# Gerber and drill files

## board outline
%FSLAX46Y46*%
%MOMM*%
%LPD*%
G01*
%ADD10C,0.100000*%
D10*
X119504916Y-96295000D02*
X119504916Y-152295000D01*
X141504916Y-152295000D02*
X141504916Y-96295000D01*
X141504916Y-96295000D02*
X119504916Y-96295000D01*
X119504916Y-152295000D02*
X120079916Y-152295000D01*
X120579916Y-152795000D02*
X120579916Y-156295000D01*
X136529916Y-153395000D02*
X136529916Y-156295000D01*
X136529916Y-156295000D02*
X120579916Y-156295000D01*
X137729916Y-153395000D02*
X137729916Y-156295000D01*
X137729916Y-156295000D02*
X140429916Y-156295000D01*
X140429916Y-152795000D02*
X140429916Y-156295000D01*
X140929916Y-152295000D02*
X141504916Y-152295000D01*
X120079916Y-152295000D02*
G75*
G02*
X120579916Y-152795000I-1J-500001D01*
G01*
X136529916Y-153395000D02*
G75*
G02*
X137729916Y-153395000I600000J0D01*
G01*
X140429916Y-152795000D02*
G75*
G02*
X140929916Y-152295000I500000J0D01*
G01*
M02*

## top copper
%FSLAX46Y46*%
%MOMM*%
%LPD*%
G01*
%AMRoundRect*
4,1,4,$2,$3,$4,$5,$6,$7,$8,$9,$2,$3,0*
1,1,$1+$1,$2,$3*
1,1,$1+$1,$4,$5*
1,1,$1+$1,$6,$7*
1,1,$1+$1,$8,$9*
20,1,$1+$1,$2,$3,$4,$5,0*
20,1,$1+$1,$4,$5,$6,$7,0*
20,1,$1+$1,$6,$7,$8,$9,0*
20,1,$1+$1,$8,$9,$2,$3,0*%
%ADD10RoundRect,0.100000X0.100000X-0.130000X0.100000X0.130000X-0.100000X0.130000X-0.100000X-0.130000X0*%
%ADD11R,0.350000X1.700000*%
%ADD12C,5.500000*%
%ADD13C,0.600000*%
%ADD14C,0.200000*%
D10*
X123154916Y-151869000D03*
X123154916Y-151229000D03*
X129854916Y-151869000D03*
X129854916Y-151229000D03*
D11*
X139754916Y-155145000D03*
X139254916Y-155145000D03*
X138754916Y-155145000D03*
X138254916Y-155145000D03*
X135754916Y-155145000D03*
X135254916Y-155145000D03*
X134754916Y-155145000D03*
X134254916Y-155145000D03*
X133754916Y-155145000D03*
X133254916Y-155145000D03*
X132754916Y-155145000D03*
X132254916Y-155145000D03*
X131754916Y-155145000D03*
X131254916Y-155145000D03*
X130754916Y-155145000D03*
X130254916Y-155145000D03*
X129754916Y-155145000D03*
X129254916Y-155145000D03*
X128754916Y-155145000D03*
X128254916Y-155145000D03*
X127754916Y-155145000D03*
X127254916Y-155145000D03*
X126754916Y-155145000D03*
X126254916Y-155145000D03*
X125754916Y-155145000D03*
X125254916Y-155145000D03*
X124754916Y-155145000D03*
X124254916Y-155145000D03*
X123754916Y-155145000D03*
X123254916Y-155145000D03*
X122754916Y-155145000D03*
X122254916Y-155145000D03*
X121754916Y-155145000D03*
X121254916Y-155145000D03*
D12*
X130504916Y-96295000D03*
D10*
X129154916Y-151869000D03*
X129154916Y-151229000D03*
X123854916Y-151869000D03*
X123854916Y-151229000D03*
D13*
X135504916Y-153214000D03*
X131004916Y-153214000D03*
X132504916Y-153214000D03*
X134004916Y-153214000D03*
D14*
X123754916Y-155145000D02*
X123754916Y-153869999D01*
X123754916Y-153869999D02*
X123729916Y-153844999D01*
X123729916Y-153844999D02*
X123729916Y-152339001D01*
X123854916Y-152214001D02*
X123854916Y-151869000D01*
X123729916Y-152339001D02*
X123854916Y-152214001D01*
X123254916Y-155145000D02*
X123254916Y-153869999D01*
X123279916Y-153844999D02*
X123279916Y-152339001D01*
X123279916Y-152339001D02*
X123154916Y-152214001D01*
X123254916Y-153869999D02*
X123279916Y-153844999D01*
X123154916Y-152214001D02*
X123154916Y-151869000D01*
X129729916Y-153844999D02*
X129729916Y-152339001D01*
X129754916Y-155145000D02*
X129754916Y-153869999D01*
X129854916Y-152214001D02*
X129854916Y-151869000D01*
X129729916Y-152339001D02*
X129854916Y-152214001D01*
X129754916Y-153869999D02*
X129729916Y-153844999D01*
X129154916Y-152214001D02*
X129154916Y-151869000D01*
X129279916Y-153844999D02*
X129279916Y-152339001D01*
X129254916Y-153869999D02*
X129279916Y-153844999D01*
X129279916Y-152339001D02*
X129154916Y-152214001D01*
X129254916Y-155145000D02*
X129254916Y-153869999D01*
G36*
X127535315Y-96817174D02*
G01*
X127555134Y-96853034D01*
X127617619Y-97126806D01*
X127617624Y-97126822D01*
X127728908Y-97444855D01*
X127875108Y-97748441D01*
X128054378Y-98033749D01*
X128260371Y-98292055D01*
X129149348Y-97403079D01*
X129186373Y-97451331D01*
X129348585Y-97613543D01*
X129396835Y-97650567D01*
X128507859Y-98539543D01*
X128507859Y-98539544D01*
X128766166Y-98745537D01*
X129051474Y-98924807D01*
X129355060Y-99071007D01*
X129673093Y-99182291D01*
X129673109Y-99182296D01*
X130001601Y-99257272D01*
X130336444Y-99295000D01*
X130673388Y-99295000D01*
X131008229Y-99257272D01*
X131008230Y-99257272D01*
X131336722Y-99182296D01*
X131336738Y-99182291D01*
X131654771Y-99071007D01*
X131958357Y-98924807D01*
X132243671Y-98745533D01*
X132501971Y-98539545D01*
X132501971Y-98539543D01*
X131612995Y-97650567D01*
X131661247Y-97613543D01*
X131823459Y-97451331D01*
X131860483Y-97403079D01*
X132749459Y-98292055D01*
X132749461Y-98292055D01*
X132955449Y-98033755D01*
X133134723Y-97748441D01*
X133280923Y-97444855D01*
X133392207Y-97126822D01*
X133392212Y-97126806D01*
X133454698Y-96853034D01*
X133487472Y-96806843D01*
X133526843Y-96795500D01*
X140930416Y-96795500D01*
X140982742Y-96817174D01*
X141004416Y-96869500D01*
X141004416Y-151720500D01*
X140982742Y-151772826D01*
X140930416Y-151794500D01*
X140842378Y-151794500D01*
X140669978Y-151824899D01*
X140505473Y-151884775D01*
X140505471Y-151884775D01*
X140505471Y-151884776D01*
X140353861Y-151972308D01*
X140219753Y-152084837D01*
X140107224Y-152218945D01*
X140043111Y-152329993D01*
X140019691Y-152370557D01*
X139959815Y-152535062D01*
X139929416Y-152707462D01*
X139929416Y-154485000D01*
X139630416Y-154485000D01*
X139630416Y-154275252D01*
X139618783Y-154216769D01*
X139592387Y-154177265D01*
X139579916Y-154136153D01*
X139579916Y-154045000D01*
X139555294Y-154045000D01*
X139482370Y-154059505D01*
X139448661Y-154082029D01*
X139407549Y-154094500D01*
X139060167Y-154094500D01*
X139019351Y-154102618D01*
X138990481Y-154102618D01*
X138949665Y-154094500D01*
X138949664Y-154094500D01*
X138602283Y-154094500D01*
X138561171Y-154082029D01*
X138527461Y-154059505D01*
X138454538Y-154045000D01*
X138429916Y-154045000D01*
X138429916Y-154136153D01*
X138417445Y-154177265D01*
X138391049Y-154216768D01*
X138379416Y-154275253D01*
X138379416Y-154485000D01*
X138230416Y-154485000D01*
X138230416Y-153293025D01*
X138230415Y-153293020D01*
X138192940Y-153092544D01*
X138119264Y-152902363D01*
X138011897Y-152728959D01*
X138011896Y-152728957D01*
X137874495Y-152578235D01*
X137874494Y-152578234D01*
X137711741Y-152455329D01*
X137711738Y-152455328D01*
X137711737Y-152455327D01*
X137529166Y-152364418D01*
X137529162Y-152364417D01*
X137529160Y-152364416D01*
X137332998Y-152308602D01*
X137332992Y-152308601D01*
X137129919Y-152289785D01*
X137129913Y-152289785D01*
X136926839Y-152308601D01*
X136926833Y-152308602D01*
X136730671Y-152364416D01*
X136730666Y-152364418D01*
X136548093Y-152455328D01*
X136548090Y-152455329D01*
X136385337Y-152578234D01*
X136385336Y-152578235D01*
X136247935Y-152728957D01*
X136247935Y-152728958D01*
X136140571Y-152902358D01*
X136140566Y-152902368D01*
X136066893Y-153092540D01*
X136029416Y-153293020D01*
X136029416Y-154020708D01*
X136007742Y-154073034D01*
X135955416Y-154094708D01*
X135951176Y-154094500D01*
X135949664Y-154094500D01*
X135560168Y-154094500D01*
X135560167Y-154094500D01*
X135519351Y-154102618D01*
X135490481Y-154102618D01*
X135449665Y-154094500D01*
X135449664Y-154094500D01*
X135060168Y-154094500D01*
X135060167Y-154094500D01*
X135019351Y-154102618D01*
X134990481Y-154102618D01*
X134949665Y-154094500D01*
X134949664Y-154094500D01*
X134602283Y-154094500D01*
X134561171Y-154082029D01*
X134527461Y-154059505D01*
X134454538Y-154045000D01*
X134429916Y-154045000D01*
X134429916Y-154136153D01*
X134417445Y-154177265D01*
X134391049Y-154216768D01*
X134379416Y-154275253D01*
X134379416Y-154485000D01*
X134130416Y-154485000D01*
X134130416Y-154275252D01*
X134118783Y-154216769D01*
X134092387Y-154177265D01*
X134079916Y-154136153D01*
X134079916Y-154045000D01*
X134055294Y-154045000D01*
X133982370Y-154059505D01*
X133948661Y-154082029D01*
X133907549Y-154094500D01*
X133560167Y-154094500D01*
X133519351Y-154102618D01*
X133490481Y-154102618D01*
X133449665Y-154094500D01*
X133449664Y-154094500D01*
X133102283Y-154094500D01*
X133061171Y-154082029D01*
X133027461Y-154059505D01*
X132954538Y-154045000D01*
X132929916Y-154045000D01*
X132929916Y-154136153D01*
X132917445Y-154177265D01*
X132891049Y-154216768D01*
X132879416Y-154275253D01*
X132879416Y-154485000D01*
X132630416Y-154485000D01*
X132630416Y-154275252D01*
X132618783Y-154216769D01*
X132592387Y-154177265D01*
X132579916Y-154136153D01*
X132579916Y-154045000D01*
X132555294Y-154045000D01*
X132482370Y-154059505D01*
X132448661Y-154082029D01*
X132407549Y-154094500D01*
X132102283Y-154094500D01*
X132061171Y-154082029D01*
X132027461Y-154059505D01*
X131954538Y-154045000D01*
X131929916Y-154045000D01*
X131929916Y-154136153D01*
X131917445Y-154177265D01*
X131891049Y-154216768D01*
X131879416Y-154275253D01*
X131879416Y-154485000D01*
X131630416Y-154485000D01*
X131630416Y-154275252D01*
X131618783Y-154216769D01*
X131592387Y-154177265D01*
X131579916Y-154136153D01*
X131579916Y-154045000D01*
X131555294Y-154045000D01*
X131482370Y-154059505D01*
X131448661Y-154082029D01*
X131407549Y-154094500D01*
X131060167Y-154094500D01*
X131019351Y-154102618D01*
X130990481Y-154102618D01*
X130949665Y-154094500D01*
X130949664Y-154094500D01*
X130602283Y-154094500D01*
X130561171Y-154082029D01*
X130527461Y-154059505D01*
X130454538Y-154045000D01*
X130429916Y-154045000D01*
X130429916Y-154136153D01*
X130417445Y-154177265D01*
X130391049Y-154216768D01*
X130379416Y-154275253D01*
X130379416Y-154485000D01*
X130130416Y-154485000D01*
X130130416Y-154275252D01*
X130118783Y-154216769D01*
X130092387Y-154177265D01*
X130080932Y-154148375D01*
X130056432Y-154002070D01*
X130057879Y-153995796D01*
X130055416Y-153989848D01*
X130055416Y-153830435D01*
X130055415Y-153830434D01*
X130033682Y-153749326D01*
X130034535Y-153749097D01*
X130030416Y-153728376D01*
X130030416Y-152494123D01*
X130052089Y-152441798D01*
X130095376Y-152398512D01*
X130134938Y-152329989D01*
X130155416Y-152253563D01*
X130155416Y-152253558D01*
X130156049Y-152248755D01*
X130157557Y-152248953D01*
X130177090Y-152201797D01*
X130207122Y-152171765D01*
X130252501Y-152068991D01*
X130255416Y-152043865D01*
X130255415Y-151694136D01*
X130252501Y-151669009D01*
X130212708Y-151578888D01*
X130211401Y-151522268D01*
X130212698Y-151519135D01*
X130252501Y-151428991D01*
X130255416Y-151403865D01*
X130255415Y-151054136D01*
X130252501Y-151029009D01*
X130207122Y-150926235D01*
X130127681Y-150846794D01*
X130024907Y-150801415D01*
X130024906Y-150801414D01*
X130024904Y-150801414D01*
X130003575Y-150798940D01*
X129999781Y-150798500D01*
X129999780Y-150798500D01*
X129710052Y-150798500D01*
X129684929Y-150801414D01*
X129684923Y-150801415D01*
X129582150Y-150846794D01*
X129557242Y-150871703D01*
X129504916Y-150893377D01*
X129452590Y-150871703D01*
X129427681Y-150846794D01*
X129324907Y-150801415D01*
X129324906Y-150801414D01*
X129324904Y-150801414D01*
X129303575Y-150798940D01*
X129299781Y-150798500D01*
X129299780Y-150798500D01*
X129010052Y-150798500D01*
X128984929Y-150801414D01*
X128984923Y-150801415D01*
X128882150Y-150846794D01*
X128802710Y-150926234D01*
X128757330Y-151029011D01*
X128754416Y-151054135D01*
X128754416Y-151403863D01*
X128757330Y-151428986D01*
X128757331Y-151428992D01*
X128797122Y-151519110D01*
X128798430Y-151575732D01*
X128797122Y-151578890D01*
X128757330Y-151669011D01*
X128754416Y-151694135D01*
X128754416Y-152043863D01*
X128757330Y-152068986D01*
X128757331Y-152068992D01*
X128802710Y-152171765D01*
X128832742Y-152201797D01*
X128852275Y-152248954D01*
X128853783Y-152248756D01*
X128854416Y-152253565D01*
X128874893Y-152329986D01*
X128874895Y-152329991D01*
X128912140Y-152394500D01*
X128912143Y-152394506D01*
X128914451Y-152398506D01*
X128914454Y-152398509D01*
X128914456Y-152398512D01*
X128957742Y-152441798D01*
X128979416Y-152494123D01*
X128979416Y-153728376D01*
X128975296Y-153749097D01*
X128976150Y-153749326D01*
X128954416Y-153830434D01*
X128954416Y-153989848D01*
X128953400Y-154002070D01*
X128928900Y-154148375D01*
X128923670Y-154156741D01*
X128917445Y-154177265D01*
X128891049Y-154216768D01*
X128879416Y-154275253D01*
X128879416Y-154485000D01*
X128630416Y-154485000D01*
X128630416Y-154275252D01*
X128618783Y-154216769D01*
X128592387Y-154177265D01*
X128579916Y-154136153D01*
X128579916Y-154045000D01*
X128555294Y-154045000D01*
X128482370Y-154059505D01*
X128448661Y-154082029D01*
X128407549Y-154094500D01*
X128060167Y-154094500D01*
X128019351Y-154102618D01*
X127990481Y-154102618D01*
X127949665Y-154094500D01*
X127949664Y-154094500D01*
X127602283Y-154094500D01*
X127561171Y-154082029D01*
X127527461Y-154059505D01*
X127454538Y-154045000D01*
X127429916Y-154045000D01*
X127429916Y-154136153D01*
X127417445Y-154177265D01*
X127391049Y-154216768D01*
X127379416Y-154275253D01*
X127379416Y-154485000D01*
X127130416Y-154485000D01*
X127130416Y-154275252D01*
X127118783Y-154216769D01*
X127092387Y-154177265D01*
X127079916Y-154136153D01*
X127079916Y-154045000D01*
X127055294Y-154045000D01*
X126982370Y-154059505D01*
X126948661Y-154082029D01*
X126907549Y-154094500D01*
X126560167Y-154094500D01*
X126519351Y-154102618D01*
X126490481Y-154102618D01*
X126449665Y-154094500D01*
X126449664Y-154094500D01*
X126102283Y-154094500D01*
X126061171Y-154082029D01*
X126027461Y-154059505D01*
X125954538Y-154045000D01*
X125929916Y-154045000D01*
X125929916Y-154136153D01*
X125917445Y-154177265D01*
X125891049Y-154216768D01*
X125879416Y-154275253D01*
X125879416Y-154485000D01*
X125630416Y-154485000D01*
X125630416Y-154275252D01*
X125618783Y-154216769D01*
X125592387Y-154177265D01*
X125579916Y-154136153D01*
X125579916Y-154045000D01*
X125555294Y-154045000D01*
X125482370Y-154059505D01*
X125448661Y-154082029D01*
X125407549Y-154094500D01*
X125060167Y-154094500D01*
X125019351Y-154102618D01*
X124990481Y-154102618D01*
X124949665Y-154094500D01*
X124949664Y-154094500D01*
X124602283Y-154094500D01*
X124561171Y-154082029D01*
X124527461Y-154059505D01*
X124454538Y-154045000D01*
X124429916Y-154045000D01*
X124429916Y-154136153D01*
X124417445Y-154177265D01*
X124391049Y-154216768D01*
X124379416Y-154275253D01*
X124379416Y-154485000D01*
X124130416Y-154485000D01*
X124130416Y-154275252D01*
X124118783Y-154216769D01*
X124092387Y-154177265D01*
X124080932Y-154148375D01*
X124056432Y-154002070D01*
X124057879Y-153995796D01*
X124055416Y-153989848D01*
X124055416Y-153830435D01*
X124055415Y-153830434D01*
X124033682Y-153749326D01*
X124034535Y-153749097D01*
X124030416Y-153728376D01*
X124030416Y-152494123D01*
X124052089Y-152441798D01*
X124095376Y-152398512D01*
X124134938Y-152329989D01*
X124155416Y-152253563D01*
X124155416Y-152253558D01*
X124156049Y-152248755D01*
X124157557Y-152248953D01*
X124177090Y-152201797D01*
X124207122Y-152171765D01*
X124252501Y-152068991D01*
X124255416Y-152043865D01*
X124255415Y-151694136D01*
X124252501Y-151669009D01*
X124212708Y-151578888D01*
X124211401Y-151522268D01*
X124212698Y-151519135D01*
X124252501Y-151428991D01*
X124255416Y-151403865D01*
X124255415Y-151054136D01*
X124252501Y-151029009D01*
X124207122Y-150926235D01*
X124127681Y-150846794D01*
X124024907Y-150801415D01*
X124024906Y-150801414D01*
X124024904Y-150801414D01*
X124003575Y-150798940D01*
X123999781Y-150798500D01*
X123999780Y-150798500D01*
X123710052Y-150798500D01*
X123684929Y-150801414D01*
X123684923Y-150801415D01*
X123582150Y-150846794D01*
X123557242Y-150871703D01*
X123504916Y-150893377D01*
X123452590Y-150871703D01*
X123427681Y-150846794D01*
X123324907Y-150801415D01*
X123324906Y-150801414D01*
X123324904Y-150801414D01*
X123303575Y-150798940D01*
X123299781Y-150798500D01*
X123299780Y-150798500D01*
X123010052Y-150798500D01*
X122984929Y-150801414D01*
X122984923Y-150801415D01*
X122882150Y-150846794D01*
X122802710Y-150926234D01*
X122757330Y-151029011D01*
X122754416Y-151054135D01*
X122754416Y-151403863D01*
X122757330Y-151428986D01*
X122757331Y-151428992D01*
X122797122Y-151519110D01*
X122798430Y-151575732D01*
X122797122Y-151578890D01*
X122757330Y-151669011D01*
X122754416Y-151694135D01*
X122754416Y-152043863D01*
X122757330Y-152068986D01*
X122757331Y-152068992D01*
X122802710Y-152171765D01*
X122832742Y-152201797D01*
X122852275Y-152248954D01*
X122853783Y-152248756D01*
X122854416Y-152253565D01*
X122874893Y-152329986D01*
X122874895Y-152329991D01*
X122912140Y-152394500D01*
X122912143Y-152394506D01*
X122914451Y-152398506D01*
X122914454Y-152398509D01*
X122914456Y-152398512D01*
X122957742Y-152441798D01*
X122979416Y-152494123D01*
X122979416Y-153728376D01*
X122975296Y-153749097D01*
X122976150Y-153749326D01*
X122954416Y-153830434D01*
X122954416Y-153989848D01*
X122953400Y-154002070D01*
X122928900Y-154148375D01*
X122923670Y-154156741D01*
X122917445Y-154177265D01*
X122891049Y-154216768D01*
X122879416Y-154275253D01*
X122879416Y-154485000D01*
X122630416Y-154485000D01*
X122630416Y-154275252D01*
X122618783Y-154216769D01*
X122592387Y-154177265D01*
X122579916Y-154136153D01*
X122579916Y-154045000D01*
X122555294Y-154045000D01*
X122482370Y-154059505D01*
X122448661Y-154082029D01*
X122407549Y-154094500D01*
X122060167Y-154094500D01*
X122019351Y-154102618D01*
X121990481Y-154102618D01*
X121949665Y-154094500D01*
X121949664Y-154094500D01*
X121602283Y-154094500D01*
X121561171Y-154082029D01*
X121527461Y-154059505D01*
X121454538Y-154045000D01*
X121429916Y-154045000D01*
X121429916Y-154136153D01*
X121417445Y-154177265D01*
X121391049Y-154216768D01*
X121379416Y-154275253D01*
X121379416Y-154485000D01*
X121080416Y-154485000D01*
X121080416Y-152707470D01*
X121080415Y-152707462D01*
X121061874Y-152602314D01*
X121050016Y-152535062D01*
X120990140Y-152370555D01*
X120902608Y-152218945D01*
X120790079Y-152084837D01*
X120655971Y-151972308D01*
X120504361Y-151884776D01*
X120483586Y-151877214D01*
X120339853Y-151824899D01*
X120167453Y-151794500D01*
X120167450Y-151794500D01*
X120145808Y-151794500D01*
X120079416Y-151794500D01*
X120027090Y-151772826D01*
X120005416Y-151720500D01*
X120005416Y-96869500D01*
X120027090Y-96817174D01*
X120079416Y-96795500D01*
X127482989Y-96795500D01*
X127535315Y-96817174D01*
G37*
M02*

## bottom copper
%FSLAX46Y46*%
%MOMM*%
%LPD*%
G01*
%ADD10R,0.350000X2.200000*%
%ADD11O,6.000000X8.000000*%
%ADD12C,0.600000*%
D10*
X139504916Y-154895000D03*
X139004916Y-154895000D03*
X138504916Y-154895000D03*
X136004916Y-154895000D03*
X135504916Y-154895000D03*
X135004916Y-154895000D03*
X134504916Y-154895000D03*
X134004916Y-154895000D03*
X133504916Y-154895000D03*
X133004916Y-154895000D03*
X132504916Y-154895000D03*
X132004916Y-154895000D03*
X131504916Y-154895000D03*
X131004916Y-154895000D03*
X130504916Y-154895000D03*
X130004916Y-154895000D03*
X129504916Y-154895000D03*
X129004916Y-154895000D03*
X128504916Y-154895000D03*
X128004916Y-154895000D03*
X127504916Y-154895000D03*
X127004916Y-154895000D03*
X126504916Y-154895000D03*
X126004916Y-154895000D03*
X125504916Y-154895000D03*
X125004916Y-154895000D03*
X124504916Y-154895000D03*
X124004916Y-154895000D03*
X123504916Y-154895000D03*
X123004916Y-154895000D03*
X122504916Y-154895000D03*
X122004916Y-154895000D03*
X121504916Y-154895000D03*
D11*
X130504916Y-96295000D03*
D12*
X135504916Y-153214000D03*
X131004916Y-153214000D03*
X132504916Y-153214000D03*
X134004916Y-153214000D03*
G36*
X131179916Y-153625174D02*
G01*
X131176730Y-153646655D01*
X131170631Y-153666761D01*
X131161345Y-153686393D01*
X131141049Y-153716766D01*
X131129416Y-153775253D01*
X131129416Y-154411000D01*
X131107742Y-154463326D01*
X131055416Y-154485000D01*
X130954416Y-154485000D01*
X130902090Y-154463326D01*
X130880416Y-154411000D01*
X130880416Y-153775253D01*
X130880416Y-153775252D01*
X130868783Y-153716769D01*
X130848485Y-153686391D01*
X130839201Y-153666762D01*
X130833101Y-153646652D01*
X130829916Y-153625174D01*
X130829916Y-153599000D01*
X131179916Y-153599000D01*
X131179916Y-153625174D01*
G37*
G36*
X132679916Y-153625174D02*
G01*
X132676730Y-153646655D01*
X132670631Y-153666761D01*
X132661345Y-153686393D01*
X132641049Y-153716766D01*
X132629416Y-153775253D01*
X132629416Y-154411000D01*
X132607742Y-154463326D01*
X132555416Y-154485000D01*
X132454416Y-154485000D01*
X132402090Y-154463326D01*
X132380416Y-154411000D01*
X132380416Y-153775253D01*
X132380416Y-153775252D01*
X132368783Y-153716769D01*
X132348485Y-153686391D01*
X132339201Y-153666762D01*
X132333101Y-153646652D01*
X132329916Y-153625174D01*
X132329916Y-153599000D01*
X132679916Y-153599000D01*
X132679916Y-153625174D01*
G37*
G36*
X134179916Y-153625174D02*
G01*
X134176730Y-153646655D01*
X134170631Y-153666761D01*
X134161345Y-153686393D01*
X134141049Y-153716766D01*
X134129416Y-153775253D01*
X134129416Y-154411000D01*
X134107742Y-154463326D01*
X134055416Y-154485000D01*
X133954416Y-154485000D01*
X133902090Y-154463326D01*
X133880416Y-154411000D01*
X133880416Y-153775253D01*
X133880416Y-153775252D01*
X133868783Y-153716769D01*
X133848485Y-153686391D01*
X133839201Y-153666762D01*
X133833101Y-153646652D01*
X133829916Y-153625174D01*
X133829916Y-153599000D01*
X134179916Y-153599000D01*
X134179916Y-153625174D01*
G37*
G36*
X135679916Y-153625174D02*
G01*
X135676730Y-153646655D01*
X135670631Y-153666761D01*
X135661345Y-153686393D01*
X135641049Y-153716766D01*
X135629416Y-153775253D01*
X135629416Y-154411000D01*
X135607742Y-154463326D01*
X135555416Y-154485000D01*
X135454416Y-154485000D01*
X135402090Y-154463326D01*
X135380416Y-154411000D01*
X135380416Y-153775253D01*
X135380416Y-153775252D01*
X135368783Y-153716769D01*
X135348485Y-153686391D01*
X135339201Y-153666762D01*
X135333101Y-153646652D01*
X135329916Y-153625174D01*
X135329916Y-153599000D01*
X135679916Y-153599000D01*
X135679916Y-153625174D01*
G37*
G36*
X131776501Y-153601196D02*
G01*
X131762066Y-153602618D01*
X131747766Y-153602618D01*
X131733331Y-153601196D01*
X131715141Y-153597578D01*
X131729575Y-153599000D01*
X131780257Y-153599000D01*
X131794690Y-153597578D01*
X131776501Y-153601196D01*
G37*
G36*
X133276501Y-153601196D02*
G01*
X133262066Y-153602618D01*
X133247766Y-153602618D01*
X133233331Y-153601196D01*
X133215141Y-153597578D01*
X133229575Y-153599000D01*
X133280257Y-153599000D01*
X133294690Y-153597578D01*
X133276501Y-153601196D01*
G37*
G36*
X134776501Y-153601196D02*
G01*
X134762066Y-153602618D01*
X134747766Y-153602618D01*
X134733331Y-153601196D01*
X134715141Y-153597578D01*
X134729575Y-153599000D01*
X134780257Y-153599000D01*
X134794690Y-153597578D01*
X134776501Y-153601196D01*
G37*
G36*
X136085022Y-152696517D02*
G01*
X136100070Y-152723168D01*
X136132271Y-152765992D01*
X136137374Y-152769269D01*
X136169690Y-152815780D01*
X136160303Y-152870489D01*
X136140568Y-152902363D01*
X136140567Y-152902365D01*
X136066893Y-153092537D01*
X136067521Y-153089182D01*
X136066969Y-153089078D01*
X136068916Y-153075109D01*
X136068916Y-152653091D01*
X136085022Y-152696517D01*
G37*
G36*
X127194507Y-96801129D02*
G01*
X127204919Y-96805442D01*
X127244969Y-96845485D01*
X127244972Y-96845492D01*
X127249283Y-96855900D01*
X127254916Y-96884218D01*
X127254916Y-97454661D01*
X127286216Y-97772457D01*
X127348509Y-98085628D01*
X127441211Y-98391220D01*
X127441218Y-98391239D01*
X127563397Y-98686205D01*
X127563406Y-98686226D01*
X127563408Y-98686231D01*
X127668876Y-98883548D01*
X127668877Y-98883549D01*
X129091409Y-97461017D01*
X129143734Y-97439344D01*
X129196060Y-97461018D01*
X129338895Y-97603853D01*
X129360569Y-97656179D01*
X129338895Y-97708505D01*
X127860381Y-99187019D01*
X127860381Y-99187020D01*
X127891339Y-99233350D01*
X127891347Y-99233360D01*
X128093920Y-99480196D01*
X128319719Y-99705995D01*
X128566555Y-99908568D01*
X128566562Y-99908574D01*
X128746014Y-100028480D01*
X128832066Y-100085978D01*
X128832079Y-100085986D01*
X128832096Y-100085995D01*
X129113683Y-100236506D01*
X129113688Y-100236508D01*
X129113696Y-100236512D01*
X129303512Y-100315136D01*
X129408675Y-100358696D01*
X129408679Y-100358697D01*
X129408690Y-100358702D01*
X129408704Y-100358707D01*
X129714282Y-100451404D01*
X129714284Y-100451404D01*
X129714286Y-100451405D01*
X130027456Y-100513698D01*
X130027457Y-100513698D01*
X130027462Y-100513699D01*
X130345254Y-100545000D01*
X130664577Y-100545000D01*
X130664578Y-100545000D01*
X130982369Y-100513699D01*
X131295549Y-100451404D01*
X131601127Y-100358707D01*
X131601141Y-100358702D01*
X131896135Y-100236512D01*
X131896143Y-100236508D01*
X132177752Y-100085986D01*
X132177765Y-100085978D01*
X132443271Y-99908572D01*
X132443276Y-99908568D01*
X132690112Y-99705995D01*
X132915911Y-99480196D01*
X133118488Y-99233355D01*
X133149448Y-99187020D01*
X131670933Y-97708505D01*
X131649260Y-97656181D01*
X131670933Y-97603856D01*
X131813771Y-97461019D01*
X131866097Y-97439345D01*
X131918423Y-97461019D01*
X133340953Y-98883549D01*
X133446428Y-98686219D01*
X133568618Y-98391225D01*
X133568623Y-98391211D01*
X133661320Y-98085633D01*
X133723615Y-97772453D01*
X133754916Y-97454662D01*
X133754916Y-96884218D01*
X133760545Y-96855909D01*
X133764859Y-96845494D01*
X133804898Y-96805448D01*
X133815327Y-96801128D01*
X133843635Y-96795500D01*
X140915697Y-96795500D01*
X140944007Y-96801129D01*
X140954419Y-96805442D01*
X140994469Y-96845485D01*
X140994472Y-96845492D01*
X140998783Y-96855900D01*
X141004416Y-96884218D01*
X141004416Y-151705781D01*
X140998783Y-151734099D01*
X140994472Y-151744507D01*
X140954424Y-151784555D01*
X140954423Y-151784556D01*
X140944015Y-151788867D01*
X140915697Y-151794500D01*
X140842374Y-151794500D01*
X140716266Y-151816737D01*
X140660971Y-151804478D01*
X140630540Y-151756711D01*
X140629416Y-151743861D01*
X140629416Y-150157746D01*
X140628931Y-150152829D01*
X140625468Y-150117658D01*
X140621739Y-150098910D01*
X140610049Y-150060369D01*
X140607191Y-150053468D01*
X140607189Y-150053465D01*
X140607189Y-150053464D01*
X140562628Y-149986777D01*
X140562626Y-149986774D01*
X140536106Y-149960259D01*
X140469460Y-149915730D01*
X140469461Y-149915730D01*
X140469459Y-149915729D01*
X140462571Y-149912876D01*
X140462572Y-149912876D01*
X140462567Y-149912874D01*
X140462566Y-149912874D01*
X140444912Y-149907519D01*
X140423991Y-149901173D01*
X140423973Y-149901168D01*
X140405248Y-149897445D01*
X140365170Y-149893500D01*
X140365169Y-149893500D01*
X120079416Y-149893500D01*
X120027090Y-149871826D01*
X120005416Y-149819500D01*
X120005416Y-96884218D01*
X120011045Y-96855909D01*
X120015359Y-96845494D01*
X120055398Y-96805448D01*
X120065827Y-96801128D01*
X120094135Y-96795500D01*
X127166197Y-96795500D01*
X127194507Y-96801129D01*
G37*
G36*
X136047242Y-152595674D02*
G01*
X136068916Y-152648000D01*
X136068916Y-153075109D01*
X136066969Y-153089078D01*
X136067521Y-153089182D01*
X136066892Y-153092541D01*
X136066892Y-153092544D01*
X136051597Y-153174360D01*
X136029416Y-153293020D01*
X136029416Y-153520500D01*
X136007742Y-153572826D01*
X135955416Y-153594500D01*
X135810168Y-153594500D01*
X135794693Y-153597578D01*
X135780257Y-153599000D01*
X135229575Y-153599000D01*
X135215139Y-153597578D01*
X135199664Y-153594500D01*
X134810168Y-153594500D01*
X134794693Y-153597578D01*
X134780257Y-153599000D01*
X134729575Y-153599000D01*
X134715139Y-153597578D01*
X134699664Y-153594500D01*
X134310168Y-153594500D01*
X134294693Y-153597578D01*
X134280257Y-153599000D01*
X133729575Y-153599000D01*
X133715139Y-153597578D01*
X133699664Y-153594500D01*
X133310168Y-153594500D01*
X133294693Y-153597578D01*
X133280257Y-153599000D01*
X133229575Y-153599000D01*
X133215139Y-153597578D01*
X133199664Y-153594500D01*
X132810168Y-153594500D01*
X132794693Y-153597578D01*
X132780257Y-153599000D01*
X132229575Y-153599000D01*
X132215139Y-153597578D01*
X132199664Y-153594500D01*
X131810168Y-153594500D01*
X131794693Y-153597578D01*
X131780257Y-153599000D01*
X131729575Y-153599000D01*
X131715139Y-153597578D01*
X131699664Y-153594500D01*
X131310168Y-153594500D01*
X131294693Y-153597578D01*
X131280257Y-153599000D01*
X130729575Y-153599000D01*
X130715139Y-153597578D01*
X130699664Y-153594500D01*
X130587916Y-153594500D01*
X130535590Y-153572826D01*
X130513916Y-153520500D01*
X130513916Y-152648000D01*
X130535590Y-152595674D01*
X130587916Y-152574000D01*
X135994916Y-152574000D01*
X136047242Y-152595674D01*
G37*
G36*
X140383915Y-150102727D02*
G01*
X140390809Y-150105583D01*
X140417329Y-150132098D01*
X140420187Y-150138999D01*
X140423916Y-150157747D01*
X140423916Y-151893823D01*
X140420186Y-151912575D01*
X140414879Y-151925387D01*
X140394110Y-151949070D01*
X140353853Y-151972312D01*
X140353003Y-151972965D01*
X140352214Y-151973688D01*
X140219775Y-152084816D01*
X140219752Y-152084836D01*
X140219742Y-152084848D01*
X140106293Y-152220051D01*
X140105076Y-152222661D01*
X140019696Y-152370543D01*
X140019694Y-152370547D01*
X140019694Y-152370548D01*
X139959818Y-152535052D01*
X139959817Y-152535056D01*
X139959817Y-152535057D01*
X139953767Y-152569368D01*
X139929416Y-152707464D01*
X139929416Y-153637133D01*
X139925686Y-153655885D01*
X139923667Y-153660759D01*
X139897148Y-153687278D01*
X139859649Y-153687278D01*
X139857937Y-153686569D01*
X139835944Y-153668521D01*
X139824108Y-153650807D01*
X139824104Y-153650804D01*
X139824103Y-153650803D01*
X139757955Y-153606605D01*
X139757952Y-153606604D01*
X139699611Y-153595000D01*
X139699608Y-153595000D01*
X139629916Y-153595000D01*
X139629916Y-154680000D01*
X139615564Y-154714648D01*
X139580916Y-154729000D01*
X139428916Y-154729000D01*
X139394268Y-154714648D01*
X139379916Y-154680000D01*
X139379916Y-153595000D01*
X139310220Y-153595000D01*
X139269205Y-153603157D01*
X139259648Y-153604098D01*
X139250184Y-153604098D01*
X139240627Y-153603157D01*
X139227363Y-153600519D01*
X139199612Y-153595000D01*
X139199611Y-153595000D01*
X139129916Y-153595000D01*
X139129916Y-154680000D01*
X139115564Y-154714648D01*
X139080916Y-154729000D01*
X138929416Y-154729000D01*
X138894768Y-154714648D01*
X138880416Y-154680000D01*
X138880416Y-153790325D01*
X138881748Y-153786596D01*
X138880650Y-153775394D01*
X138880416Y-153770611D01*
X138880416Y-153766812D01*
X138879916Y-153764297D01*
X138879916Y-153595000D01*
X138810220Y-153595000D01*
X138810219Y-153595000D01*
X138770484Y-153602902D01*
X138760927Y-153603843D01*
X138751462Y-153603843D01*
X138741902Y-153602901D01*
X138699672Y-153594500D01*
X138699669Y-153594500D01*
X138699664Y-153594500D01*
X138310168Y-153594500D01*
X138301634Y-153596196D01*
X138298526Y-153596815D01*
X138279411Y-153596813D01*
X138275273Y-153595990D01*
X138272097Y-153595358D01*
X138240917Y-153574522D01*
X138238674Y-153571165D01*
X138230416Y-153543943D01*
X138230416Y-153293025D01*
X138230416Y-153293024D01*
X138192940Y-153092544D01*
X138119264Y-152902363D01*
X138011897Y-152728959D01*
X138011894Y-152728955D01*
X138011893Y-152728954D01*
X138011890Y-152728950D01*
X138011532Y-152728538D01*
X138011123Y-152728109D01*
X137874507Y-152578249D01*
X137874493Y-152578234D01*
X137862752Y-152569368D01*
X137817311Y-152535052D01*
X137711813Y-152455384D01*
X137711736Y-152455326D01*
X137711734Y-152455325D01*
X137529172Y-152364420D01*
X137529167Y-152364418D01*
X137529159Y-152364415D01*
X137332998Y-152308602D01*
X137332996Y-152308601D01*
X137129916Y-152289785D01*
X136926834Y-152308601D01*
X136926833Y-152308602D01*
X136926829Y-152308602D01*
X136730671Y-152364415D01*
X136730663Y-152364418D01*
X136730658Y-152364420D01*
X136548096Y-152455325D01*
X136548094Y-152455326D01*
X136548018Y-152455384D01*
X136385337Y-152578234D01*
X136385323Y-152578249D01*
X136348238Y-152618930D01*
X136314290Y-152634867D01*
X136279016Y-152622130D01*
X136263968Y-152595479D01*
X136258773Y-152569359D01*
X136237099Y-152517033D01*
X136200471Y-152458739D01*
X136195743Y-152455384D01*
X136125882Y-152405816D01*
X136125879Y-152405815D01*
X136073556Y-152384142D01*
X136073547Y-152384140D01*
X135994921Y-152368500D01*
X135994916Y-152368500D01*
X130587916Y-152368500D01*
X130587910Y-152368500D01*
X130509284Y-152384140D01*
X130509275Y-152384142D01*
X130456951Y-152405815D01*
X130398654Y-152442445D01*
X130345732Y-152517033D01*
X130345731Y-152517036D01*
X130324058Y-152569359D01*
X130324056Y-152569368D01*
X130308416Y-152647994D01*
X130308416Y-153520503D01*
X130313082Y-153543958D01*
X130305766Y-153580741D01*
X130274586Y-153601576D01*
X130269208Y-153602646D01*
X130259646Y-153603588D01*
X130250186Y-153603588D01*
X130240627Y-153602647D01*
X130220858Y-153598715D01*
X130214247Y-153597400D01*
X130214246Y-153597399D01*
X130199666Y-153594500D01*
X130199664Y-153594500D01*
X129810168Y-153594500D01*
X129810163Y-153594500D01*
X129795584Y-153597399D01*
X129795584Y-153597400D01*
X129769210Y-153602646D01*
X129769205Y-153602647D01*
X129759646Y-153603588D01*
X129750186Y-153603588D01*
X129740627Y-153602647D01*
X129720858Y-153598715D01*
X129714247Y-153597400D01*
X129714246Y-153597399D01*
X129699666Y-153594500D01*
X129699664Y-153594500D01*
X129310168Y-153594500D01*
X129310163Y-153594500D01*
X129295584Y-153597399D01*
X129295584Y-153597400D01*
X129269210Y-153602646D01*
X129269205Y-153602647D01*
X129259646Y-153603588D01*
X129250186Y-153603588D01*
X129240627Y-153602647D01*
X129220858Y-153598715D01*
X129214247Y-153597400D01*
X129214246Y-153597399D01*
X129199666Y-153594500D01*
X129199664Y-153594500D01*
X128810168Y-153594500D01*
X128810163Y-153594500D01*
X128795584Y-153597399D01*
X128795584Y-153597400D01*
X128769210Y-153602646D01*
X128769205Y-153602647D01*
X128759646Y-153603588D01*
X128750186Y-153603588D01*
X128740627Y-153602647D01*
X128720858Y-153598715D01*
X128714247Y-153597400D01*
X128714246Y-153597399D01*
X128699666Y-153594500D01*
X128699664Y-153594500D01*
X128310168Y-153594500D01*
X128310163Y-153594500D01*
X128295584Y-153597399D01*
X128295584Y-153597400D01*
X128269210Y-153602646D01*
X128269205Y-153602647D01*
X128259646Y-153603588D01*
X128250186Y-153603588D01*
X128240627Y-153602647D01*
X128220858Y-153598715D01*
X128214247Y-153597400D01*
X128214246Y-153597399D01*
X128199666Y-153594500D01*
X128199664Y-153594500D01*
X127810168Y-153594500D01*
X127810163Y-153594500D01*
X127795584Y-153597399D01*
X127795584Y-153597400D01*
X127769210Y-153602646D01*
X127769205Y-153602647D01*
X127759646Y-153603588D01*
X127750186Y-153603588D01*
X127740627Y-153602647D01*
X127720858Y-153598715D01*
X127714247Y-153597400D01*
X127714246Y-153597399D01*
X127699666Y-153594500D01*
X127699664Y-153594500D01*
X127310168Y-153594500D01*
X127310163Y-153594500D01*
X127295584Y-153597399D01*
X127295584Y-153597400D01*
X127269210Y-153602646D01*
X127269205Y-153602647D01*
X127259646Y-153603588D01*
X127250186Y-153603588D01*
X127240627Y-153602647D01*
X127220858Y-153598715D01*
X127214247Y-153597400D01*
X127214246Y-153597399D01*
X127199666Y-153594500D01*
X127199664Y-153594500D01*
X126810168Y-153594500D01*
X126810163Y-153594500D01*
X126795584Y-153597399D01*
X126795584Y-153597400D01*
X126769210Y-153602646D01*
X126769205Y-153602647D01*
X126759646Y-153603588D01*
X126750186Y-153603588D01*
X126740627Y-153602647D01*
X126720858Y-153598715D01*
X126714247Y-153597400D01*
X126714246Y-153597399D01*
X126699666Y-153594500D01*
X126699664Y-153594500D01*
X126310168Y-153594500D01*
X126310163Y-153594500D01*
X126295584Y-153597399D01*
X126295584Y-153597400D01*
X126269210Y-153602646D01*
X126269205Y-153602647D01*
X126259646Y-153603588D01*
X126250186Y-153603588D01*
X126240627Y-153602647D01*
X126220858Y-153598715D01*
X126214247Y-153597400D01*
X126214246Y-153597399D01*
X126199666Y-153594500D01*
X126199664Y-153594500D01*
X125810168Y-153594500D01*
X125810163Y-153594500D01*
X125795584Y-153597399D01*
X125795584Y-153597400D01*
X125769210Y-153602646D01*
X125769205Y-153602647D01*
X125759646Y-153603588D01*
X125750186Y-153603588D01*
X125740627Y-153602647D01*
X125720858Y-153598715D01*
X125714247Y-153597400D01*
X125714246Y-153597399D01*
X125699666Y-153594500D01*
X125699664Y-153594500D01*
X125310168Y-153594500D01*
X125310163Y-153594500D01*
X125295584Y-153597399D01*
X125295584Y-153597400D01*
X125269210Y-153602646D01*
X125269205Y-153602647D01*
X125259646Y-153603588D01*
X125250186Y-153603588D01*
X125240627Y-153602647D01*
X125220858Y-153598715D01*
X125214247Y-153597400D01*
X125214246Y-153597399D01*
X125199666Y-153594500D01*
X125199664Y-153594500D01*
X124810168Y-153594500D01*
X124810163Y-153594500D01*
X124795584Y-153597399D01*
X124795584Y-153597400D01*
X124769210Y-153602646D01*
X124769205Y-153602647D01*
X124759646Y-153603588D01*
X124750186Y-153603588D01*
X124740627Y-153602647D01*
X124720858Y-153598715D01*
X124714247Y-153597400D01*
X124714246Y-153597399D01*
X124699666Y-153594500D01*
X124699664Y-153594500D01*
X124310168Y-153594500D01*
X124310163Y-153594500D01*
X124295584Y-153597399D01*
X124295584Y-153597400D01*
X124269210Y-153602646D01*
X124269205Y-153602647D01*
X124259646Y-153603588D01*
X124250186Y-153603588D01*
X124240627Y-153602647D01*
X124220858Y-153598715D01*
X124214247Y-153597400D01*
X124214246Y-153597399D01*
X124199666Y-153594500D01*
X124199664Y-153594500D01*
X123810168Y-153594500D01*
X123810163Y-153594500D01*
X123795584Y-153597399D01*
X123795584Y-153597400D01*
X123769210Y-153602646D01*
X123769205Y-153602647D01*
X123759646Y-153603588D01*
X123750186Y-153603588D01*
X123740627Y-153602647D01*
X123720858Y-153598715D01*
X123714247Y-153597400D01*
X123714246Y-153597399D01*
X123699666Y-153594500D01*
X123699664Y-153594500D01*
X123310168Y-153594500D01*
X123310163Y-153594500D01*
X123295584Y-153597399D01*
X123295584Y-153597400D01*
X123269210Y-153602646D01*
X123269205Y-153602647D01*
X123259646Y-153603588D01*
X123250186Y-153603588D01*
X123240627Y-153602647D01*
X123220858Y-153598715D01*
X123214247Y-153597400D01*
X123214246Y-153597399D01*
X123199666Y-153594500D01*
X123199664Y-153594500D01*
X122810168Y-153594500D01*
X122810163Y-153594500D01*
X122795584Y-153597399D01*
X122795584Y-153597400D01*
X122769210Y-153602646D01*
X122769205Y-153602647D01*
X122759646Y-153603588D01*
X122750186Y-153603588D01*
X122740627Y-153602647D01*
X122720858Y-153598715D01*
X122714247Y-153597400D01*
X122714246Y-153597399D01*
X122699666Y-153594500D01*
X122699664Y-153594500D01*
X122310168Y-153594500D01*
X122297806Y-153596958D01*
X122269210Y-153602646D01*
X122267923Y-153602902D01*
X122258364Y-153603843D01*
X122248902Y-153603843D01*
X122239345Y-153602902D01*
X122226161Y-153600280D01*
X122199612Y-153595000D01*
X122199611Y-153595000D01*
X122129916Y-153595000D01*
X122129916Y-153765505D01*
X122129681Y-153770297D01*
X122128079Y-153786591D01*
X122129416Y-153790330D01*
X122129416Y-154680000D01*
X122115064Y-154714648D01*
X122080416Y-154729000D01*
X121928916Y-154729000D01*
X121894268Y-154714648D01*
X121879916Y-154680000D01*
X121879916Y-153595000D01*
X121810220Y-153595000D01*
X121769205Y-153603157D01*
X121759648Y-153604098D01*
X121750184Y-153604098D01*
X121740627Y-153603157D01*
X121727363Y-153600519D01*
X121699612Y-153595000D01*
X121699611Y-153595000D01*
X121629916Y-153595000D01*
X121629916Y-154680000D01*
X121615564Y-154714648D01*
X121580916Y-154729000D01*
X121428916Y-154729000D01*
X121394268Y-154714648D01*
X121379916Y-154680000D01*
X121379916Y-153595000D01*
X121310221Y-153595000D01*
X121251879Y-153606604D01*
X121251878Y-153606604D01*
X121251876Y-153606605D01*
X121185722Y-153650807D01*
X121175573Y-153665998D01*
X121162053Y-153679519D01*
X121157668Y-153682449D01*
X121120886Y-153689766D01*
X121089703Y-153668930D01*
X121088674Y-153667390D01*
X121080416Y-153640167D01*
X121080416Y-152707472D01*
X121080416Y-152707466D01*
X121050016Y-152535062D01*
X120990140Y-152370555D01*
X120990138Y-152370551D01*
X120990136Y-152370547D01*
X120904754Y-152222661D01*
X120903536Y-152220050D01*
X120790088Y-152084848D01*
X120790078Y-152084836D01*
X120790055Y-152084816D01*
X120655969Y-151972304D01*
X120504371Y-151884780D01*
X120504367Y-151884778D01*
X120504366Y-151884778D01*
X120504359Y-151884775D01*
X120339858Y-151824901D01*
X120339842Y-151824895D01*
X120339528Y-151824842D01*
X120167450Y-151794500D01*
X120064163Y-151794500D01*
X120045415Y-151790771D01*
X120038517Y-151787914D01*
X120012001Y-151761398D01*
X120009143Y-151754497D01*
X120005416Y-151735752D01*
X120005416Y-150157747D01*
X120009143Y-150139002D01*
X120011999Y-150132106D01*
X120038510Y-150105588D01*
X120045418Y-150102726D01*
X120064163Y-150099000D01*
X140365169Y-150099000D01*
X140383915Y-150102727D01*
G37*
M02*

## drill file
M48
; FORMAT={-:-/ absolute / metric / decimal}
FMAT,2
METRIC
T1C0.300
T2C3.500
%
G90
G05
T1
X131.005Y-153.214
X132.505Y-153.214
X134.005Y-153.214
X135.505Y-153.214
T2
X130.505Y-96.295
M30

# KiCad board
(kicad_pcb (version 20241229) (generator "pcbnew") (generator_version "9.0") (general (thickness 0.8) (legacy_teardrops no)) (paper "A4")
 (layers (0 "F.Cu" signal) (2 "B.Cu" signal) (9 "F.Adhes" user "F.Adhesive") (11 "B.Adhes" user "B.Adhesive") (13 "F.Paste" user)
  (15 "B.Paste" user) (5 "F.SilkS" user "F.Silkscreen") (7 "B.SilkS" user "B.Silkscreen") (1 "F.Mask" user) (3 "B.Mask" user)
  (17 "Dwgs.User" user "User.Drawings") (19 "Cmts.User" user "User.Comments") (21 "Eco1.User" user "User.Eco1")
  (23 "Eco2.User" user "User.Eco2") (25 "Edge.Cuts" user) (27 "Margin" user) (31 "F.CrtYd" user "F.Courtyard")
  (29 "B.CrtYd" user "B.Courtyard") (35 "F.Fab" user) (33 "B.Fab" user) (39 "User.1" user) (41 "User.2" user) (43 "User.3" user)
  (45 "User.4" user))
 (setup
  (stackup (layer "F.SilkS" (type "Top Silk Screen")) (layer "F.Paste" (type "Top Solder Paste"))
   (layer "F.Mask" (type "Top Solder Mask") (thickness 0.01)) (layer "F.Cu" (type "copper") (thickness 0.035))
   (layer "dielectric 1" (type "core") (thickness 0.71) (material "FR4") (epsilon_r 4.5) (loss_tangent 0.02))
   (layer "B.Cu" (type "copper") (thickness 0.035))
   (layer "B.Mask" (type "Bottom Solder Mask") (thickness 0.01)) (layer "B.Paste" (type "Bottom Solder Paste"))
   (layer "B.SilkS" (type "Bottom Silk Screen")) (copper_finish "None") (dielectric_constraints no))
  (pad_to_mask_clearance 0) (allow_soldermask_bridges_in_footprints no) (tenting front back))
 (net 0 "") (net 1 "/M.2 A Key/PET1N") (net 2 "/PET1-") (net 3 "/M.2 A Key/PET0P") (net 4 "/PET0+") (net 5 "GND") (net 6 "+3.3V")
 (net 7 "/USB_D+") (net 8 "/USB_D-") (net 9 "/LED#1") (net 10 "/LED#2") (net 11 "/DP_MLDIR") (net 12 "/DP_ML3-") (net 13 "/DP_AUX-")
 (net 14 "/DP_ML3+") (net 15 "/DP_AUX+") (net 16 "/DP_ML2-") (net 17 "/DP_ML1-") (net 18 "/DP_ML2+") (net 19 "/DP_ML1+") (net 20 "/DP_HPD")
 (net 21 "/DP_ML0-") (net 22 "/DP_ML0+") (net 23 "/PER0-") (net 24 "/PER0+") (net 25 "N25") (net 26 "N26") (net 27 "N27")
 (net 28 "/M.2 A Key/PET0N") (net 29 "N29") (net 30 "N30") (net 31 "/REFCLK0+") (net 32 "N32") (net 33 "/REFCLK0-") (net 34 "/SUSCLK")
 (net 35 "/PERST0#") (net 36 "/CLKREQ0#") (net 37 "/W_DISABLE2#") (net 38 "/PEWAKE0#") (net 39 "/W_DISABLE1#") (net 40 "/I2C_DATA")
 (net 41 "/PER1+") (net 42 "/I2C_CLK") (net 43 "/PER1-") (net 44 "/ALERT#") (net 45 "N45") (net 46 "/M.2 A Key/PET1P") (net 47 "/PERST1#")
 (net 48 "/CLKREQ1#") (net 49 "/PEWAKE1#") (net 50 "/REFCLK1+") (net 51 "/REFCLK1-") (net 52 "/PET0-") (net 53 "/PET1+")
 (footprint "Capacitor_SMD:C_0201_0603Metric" (layer "F.Cu") (at 123.154916 151.549 90)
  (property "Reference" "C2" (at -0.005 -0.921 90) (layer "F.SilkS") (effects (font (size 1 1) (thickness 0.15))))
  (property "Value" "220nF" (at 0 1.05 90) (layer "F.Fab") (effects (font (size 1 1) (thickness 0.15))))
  (pad "" smd roundrect (at -0.345 0 90) (size 0.318 0.36) (layers "F.Paste") (roundrect_rratio 0.25))
  (pad "" smd roundrect (at 0.345 0 90) (size 0.318 0.36) (layers "F.Paste") (roundrect_rratio 0.25))
  (pad "1" smd roundrect (at -0.32 0 90) (size 0.46 0.4) (layers "F.Cu" "F.Mask") (roundrect_rratio 0.25) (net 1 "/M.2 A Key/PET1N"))
  (pad "2" smd roundrect (at 0.32 0 90) (size 0.46 0.4) (layers "F.Cu" "F.Mask") (roundrect_rratio 0.25) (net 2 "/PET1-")))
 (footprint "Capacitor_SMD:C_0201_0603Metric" (layer "F.Cu") (at 129.854916 151.549 90)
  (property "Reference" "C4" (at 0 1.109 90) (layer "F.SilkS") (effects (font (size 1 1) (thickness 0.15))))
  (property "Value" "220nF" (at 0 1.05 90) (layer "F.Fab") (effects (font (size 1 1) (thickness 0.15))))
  (pad "" smd roundrect (at -0.345 0 90) (size 0.318 0.36) (layers "F.Paste") (roundrect_rratio 0.25))
  (pad "" smd roundrect (at 0.345 0 90) (size 0.318 0.36) (layers "F.Paste") (roundrect_rratio 0.25))
  (pad "1" smd roundrect (at -0.32 0 90) (size 0.46 0.4) (layers "F.Cu" "F.Mask") (roundrect_rratio 0.25) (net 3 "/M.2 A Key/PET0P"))
  (pad "2" smd roundrect (at 0.32 0 90) (size 0.46 0.4) (layers "F.Cu" "F.Mask") (roundrect_rratio 0.25) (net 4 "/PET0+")))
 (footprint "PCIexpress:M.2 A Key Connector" (layer "F.Cu") (at 130.504916 155.185)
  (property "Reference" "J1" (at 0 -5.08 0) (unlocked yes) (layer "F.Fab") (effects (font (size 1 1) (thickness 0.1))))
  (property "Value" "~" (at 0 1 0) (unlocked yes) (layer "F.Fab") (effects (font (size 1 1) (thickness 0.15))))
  (fp_line (start -11 -2.89) (end -10.425 -2.89) (stroke (width 0.1) (type default)) (layer "Edge.Cuts"))
  (fp_line (start -9.925 -2.39) (end -9.925 1.11) (stroke (width 0.1) (type default)) (layer "Edge.Cuts"))
  (fp_line (start 6.025 -1.79) (end 6.025 1.11) (stroke (width 0.1) (type default)) (layer "Edge.Cuts"))
  (fp_line (start 6.025 1.11) (end -9.925 1.11) (stroke (width 0.1) (type default)) (layer "Edge.Cuts"))
  (fp_line (start 7.225 -1.79) (end 7.225 1.11) (stroke (width 0.1) (type default)) (layer "Edge.Cuts"))
  (fp_line (start 7.225 1.11) (end 9.925 1.11) (stroke (width 0.1) (type default)) (layer "Edge.Cuts"))
  (fp_line (start 9.925 -2.39) (end 9.925 1.11) (stroke (width 0.1) (type default)) (layer "Edge.Cuts"))
  (fp_line (start 10.425 -2.89) (end 11 -2.89) (stroke (width 0.1) (type default)) (layer "Edge.Cuts"))
  (fp_arc (start -10.425 -2.89) (mid -10.071447 -2.743553) (end -9.925 -2.39) (stroke (width 0.1) (type default)) (layer "Edge.Cuts"))
  (fp_arc (start 6.025 -1.79) (mid 6.625 -2.39) (end 7.225 -1.79) (stroke (width 0.1) (type default)) (layer "Edge.Cuts"))
  (fp_arc (start 9.925 -2.39) (mid 10.071447 -2.743553) (end 10.425 -2.89) (stroke (width 0.1) (type default)) (layer "Edge.Cuts"))
  (pad "1" smd rect (at 9.25 -0.04 180) (size 0.35 1.7) (layers "F.Cu") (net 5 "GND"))
  (pad "2" smd rect (at 9 -0.29 180) (size 0.35 2.2) (layers "B.Cu") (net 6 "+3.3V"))
  (pad "3" smd rect (at 8.75 -0.04 180) (size 0.35 1.7) (layers "F.Cu") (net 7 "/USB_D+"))
  (pad "4" smd rect (at 8.5 -0.29 180) (size 0.35 2.2) (layers "B.Cu") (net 6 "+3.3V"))
  (pad "5" smd rect (at 8.25 -0.04 180) (size 0.35 1.7) (layers "F.Cu") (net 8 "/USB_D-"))
  (pad "6" smd rect (at 8 -0.29 180) (size 0.35 2.2) (layers "B.Cu") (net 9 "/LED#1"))
  (pad "7" smd rect (at 7.75 -0.04 180) (size 0.35 1.7) (layers "F.Cu") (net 5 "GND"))
  (pad "16" smd rect (at 5.5 -0.29 180) (size 0.35 2.2) (layers "B.Cu") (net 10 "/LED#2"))
  (pad "17" smd rect (at 5.25 -0.04 180) (size 0.35 1.7) (layers "F.Cu") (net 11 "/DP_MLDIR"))
  (pad "18" smd rect (at 5 -0.29 180) (size 0.35 2.2) (layers "B.Cu") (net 5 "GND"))
  (pad "19" smd rect (at 4.75 -0.04 180) (size 0.35 1.7) (layers "F.Cu") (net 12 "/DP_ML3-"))
  (pad "20" smd rect (at 4.5 -0.29 180) (size 0.35 2.2) (layers "B.Cu") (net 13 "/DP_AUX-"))
  (pad "21" smd rect (at 4.25 -0.04 180) (size 0.35 1.7) (layers "F.Cu") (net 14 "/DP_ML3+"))
  (pad "22" smd rect (at 4 -0.29 180) (size 0.35 2.2) (layers "B.Cu") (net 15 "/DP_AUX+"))
  (pad "23" smd rect (at 3.75 -0.04 180) (size 0.35 1.7) (layers "F.Cu") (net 5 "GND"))
  (pad "24" smd rect (at 3.5 -0.29 180) (size 0.35 2.2) (layers "B.Cu") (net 5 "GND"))
  (pad "25" smd rect (at 3.25 -0.04 180) (size 0.35 1.7) (layers "F.Cu") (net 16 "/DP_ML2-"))
  (pad "26" smd rect (at 3 -0.29 180) (size 0.35 2.2) (layers "B.Cu") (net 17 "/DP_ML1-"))
  (pad "27" smd rect (at 2.75 -0.04 180) (size 0.35 1.7) (layers "F.Cu") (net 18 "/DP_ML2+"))
  (pad "28" smd rect (at 2.5 -0.29 180) (size 0.35 2.2) (layers "B.Cu") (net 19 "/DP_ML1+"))
  (pad "29" smd rect (at 2.25 -0.04 180) (size 0.35 1.7) (layers "F.Cu") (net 5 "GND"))
  (pad "30" smd rect (at 2 -0.29 180) (size 0.35 2.2) (layers "B.Cu") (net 5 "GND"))
  (pad "31" smd rect (at 1.75 -0.04 180) (size 0.35 1.7) (layers "F.Cu") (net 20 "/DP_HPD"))
  (pad "32" smd rect (at 1.5 -0.29 180) (size 0.35 2.2) (layers "B.Cu") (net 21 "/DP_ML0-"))
  (pad "33" smd rect (at 1.25 -0.04 180) (size 0.35 1.7) (layers "F.Cu") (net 5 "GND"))
  (pad "34" smd rect (at 1 -0.29 180) (size 0.35 2.2) (layers "B.Cu") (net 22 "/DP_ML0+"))
  (pad "35" smd rect (at 0.75 -0.04 180) (size 0.35 1.7) (layers "F.Cu") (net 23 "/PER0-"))
  (pad "36" smd rect (at 0.5 -0.29 180) (size 0.35 2.2) (layers "B.Cu") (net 5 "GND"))
  (pad "37" smd rect (at 0.25 -0.04 180) (size 0.35 1.7) (layers "F.Cu") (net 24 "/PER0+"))
  (pad "38" smd rect (at 0 -0.29 180) (size 0.35 2.2) (layers "B.Cu") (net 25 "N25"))
  (pad "39" smd rect (at -0.25 -0.04 180) (size 0.35 1.7) (layers "F.Cu") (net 5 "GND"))
  (pad "40" smd rect (at -0.5 -0.29 180) (size 0.35 2.2) (layers "B.Cu") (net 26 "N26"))
  (pad "41" smd rect (at -0.75 -0.04 180) (size 0.35 1.7) (layers "F.Cu") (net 3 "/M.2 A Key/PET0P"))
  (pad "42" smd rect (at -1 -0.29 180) (size 0.35 2.2) (layers "B.Cu") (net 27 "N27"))
  (pad "43" smd rect (at -1.25 -0.04 180) (size 0.35 1.7) (layers "F.Cu") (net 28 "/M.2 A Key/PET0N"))
  (pad "44" smd rect (at -1.5 -0.29 180) (size 0.35 2.2) (layers "B.Cu") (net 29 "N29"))
  (pad "45" smd rect (at -1.75 -0.04 180) (size 0.35 1.7) (layers "F.Cu") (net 5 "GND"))
  (pad "46" smd rect (at -2 -0.29 180) (size 0.35 2.2) (layers "B.Cu") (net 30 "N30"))
  (pad "47" smd rect (at -2.25 -0.04 180) (size 0.35 1.7) (layers "F.Cu") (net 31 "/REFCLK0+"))
  (pad "48" smd rect (at -2.5 -0.29 180) (size 0.35 2.2) (layers "B.Cu") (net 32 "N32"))
  (pad "49" smd rect (at -2.75 -0.04 180) (size 0.35 1.7) (layers "F.Cu") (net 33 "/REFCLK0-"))
  (pad "50" smd rect (at -3 -0.29 180) (size 0.35 2.2) (layers "B.Cu") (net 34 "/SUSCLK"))
  (pad "51" smd rect (at -3.25 -0.04 180) (size 0.35 1.7) (layers "F.Cu") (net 5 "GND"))
  (pad "52" smd rect (at -3.5 -0.29 180) (size 0.35 2.2) (layers "B.Cu") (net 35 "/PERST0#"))
  (pad "53" smd rect (at -3.75 -0.04 180) (size 0.35 1.7) (layers "F.Cu") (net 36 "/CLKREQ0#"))
  (pad "54" smd rect (at -4 -0.29 180) (size 0.35 2.2) (layers "B.Cu") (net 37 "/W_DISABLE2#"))
  (pad "55" smd rect (at -4.25 -0.04 180) (size 0.35 1.7) (layers "F.Cu") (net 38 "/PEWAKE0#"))
  (pad "56" smd rect (at -4.5 -0.29 180) (size 0.35 2.2) (layers "B.Cu") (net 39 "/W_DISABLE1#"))
  (pad "57" smd rect (at -4.75 -0.04 180) (size 0.35 1.7) (layers "F.Cu") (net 5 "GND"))
  (pad "58" smd rect (at -5 -0.29 180) (size 0.35 2.2) (layers "B.Cu") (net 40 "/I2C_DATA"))
  (pad "59" smd rect (at -5.25 -0.04 180) (size 0.35 1.7) (layers "F.Cu") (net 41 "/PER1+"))
  (pad "60" smd rect (at -5.5 -0.29 180) (size 0.35 2.2) (layers "B.Cu") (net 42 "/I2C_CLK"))
  (pad "61" smd rect (at -5.75 -0.04 180) (size 0.35 1.7) (layers "F.Cu") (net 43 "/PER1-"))
  (pad "62" smd rect (at -6 -0.29 180) (size 0.35 2.2) (layers "B.Cu") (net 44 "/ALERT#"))
  (pad "63" smd rect (at -6.25 -0.04 180) (size 0.35 1.7) (layers "F.Cu") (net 5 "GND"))
  (pad "64" smd rect (at -6.5 -0.29 180) (size 0.35 2.2) (layers "B.Cu") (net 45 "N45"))
  (pad "65" smd rect (at -6.75 -0.04 180) (size 0.35 1.7) (layers "F.Cu") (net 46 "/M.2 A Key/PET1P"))
  (pad "66" smd rect (at -7 -0.29 180) (size 0.35 2.2) (layers "B.Cu") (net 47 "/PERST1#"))
  (pad "67" smd rect (at -7.25 -0.04 180) (size 0.35 1.7) (layers "F.Cu") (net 1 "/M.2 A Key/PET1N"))
  (pad "68" smd rect (at -7.5 -0.29 180) (size 0.35 2.2) (layers "B.Cu") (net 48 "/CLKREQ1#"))
  (pad "69" smd rect (at -7.75 -0.04 180) (size 0.35 1.7) (layers "F.Cu") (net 5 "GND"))
  (pad "70" smd rect (at -8 -0.29 180) (size 0.35 2.2) (layers "B.Cu") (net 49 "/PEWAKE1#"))
  (pad "71" smd rect (at -8.25 -0.04 180) (size 0.35 1.7) (layers "F.Cu") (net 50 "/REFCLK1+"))
  (pad "72" smd rect (at -8.5 -0.29 180) (size 0.35 2.2) (layers "B.Cu") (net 6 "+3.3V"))
  (pad "73" smd rect (at -8.75 -0.04 180) (size 0.35 1.7) (layers "F.Cu") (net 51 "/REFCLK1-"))
  (pad "74" smd rect (at -9 -0.29 180) (size 0.35 2.2) (layers "B.Cu") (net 6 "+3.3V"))
  (pad "75" smd rect (at -9.25 -0.04 180) (size 0.35 1.7) (layers "F.Cu") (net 5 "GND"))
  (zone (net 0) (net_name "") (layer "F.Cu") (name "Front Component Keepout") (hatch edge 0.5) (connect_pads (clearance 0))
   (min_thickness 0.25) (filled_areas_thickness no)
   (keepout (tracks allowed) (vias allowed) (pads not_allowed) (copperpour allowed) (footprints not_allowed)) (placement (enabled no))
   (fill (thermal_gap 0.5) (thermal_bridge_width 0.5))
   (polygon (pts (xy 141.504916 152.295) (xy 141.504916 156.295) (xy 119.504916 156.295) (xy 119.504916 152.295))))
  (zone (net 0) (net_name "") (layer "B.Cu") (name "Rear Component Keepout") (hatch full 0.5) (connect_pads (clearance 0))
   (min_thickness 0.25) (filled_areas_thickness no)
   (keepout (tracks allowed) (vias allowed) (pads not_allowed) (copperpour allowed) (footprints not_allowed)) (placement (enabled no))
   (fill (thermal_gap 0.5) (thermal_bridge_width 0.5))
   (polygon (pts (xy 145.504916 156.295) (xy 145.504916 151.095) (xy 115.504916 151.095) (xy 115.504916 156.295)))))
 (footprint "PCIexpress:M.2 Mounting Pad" (layer "F.Cu") (at 130.504916 126.295)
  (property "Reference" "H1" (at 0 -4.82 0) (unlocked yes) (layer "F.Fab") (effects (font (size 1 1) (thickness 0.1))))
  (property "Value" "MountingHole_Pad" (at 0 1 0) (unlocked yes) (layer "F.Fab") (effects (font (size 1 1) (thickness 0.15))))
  (pad "1" thru_hole circle (at 0 -30) (size 5.5 5.5) (drill 3.5) (layers "*.Cu" "*.Mask") (remove_unused_layers no) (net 5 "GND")
   (padstack (mode front_inner_back)
    (layer "Inner" (shape circle) (size 5.5 5.5) (zone_connect -1))
    (layer "B.Cu" (shape oval) (size 6 8) (thermal_bridge_angle 45) (zone_connect -1)))))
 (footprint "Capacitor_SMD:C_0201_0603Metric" (layer "F.Cu") (at 129.154916 151.549 90)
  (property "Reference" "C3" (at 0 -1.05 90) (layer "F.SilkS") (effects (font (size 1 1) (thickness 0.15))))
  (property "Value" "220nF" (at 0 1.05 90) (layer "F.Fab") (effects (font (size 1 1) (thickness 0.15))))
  (pad "" smd roundrect (at -0.345 0 90) (size 0.318 0.36) (layers "F.Paste") (roundrect_rratio 0.25))
  (pad "" smd roundrect (at 0.345 0 90) (size 0.318 0.36) (layers "F.Paste") (roundrect_rratio 0.25))
  (pad "1" smd roundrect (at -0.32 0 90) (size 0.46 0.4) (layers "F.Cu" "F.Mask") (roundrect_rratio 0.25) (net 28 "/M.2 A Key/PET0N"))
  (pad "2" smd roundrect (at 0.32 0 90) (size 0.46 0.4) (layers "F.Cu" "F.Mask") (roundrect_rratio 0.25) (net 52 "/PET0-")))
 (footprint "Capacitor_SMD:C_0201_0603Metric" (layer "F.Cu") (at 123.854916 151.549 90)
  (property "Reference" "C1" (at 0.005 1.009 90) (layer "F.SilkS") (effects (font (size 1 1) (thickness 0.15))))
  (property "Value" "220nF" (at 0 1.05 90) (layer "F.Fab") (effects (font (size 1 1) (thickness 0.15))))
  (pad "" smd roundrect (at -0.345 0 90) (size 0.318 0.36) (layers "F.Paste") (roundrect_rratio 0.25))
  (pad "" smd roundrect (at 0.345 0 90) (size 0.318 0.36) (layers "F.Paste") (roundrect_rratio 0.25))
  (pad "1" smd roundrect (at -0.32 0 90) (size 0.46 0.4) (layers "F.Cu" "F.Mask") (roundrect_rratio 0.25) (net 46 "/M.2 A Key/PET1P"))
  (pad "2" smd roundrect (at 0.32 0 90) (size 0.46 0.4) (layers "F.Cu" "F.Mask") (roundrect_rratio 0.25) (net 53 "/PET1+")))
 (gr_line (start 119.504916 96.295) (end 119.504916 152.295) (stroke (width 0.1) (type default)) (layer "Edge.Cuts"))
 (gr_line (start 141.504916 152.295) (end 141.504916 96.295) (stroke (width 0.1) (type default)) (layer "Edge.Cuts"))
 (gr_line (start 141.504916 96.295) (end 119.504916 96.295) (stroke (width 0.1) (type solid)) (layer "Edge.Cuts"))
 (via (at 135.504916 153.214) (size 0.6) (drill 0.3) (layers "F.Cu" "B.Cu") (free yes) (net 5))
 (via (at 131.004916 153.214) (size 0.6) (drill 0.3) (layers "F.Cu" "B.Cu") (free yes) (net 5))
 (via (at 132.504916 153.214) (size 0.6) (drill 0.3) (layers "F.Cu" "B.Cu") (free yes) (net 5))
 (via (at 134.004916 153.214) (size 0.6) (drill 0.3) (layers "F.Cu" "B.Cu") (free yes) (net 5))
 (segment (start 123.754916 155.145) (end 123.754916 153.869999) (width 0.2) (layer "F.Cu") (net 46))
 (segment (start 123.754916 153.869999) (end 123.729916 153.844999) (width 0.2) (layer "F.Cu") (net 46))
 (segment (start 123.729916 153.844999) (end 123.729916 152.339001) (width 0.2) (layer "F.Cu") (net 46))
 (segment (start 123.854916 152.214001) (end 123.854916 151.869) (width 0.2) (layer "F.Cu") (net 46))
 (segment (start 123.729916 152.339001) (end 123.854916 152.214001) (width 0.2) (layer "F.Cu") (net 46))
 (segment (start 123.254916 155.145) (end 123.254916 153.869999) (width 0.2) (layer "F.Cu") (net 1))
 (segment (start 123.279916 153.844999) (end 123.279916 152.339001) (width 0.2) (layer "F.Cu") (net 1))
 (segment (start 123.279916 152.339001) (end 123.154916 152.214001) (width 0.2) (layer "F.Cu") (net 1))
 (segment (start 123.254916 153.869999) (end 123.279916 153.844999) (width 0.2) (layer "F.Cu") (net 1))
 (segment (start 123.154916 152.214001) (end 123.154916 151.869) (width 0.2) (layer "F.Cu") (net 1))
 (segment (start 129.729916 153.844999) (end 129.729916 152.339001) (width 0.2) (layer "F.Cu") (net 3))
 (segment (start 129.754916 155.145) (end 129.754916 153.869999) (width 0.2) (layer "F.Cu") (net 3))
 (segment (start 129.854916 152.214001) (end 129.854916 151.869) (width 0.2) (layer "F.Cu") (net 3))
 (segment (start 129.729916 152.339001) (end 129.854916 152.214001) (width 0.2) (layer "F.Cu") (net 3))
 (segment (start 129.754916 153.869999) (end 129.729916 153.844999) (width 0.2) (layer "F.Cu") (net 3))
 (segment (start 129.154916 152.214001) (end 129.154916 151.869) (width 0.2) (layer "F.Cu") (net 28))
 (segment (start 129.279916 153.844999) (end 129.279916 152.339001) (width 0.2) (layer "F.Cu") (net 28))
 (segment (start 129.254916 153.869999) (end 129.279916 153.844999) (width 0.2) (layer "F.Cu") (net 28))
 (segment (start 129.279916 152.339001) (end 129.154916 152.214001) (width 0.2) (layer "F.Cu") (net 28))
 (segment (start 129.254916 155.145) (end 129.254916 153.869999) (width 0.2) (layer "F.Cu") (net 28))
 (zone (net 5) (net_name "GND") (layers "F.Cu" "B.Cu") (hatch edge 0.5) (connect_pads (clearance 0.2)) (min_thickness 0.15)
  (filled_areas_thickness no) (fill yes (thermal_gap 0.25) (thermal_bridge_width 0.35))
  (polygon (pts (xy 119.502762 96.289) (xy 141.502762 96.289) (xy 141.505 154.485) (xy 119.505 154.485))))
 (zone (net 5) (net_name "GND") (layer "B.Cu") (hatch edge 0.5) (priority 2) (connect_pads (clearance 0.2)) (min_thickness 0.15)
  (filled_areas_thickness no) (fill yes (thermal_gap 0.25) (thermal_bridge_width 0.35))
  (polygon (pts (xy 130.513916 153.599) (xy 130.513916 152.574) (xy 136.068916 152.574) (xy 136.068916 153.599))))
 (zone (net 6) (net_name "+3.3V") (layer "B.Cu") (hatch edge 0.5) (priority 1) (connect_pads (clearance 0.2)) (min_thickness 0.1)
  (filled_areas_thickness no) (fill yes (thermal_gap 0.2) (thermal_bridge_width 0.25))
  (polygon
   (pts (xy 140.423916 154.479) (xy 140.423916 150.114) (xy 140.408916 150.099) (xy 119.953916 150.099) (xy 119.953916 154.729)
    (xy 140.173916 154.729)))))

